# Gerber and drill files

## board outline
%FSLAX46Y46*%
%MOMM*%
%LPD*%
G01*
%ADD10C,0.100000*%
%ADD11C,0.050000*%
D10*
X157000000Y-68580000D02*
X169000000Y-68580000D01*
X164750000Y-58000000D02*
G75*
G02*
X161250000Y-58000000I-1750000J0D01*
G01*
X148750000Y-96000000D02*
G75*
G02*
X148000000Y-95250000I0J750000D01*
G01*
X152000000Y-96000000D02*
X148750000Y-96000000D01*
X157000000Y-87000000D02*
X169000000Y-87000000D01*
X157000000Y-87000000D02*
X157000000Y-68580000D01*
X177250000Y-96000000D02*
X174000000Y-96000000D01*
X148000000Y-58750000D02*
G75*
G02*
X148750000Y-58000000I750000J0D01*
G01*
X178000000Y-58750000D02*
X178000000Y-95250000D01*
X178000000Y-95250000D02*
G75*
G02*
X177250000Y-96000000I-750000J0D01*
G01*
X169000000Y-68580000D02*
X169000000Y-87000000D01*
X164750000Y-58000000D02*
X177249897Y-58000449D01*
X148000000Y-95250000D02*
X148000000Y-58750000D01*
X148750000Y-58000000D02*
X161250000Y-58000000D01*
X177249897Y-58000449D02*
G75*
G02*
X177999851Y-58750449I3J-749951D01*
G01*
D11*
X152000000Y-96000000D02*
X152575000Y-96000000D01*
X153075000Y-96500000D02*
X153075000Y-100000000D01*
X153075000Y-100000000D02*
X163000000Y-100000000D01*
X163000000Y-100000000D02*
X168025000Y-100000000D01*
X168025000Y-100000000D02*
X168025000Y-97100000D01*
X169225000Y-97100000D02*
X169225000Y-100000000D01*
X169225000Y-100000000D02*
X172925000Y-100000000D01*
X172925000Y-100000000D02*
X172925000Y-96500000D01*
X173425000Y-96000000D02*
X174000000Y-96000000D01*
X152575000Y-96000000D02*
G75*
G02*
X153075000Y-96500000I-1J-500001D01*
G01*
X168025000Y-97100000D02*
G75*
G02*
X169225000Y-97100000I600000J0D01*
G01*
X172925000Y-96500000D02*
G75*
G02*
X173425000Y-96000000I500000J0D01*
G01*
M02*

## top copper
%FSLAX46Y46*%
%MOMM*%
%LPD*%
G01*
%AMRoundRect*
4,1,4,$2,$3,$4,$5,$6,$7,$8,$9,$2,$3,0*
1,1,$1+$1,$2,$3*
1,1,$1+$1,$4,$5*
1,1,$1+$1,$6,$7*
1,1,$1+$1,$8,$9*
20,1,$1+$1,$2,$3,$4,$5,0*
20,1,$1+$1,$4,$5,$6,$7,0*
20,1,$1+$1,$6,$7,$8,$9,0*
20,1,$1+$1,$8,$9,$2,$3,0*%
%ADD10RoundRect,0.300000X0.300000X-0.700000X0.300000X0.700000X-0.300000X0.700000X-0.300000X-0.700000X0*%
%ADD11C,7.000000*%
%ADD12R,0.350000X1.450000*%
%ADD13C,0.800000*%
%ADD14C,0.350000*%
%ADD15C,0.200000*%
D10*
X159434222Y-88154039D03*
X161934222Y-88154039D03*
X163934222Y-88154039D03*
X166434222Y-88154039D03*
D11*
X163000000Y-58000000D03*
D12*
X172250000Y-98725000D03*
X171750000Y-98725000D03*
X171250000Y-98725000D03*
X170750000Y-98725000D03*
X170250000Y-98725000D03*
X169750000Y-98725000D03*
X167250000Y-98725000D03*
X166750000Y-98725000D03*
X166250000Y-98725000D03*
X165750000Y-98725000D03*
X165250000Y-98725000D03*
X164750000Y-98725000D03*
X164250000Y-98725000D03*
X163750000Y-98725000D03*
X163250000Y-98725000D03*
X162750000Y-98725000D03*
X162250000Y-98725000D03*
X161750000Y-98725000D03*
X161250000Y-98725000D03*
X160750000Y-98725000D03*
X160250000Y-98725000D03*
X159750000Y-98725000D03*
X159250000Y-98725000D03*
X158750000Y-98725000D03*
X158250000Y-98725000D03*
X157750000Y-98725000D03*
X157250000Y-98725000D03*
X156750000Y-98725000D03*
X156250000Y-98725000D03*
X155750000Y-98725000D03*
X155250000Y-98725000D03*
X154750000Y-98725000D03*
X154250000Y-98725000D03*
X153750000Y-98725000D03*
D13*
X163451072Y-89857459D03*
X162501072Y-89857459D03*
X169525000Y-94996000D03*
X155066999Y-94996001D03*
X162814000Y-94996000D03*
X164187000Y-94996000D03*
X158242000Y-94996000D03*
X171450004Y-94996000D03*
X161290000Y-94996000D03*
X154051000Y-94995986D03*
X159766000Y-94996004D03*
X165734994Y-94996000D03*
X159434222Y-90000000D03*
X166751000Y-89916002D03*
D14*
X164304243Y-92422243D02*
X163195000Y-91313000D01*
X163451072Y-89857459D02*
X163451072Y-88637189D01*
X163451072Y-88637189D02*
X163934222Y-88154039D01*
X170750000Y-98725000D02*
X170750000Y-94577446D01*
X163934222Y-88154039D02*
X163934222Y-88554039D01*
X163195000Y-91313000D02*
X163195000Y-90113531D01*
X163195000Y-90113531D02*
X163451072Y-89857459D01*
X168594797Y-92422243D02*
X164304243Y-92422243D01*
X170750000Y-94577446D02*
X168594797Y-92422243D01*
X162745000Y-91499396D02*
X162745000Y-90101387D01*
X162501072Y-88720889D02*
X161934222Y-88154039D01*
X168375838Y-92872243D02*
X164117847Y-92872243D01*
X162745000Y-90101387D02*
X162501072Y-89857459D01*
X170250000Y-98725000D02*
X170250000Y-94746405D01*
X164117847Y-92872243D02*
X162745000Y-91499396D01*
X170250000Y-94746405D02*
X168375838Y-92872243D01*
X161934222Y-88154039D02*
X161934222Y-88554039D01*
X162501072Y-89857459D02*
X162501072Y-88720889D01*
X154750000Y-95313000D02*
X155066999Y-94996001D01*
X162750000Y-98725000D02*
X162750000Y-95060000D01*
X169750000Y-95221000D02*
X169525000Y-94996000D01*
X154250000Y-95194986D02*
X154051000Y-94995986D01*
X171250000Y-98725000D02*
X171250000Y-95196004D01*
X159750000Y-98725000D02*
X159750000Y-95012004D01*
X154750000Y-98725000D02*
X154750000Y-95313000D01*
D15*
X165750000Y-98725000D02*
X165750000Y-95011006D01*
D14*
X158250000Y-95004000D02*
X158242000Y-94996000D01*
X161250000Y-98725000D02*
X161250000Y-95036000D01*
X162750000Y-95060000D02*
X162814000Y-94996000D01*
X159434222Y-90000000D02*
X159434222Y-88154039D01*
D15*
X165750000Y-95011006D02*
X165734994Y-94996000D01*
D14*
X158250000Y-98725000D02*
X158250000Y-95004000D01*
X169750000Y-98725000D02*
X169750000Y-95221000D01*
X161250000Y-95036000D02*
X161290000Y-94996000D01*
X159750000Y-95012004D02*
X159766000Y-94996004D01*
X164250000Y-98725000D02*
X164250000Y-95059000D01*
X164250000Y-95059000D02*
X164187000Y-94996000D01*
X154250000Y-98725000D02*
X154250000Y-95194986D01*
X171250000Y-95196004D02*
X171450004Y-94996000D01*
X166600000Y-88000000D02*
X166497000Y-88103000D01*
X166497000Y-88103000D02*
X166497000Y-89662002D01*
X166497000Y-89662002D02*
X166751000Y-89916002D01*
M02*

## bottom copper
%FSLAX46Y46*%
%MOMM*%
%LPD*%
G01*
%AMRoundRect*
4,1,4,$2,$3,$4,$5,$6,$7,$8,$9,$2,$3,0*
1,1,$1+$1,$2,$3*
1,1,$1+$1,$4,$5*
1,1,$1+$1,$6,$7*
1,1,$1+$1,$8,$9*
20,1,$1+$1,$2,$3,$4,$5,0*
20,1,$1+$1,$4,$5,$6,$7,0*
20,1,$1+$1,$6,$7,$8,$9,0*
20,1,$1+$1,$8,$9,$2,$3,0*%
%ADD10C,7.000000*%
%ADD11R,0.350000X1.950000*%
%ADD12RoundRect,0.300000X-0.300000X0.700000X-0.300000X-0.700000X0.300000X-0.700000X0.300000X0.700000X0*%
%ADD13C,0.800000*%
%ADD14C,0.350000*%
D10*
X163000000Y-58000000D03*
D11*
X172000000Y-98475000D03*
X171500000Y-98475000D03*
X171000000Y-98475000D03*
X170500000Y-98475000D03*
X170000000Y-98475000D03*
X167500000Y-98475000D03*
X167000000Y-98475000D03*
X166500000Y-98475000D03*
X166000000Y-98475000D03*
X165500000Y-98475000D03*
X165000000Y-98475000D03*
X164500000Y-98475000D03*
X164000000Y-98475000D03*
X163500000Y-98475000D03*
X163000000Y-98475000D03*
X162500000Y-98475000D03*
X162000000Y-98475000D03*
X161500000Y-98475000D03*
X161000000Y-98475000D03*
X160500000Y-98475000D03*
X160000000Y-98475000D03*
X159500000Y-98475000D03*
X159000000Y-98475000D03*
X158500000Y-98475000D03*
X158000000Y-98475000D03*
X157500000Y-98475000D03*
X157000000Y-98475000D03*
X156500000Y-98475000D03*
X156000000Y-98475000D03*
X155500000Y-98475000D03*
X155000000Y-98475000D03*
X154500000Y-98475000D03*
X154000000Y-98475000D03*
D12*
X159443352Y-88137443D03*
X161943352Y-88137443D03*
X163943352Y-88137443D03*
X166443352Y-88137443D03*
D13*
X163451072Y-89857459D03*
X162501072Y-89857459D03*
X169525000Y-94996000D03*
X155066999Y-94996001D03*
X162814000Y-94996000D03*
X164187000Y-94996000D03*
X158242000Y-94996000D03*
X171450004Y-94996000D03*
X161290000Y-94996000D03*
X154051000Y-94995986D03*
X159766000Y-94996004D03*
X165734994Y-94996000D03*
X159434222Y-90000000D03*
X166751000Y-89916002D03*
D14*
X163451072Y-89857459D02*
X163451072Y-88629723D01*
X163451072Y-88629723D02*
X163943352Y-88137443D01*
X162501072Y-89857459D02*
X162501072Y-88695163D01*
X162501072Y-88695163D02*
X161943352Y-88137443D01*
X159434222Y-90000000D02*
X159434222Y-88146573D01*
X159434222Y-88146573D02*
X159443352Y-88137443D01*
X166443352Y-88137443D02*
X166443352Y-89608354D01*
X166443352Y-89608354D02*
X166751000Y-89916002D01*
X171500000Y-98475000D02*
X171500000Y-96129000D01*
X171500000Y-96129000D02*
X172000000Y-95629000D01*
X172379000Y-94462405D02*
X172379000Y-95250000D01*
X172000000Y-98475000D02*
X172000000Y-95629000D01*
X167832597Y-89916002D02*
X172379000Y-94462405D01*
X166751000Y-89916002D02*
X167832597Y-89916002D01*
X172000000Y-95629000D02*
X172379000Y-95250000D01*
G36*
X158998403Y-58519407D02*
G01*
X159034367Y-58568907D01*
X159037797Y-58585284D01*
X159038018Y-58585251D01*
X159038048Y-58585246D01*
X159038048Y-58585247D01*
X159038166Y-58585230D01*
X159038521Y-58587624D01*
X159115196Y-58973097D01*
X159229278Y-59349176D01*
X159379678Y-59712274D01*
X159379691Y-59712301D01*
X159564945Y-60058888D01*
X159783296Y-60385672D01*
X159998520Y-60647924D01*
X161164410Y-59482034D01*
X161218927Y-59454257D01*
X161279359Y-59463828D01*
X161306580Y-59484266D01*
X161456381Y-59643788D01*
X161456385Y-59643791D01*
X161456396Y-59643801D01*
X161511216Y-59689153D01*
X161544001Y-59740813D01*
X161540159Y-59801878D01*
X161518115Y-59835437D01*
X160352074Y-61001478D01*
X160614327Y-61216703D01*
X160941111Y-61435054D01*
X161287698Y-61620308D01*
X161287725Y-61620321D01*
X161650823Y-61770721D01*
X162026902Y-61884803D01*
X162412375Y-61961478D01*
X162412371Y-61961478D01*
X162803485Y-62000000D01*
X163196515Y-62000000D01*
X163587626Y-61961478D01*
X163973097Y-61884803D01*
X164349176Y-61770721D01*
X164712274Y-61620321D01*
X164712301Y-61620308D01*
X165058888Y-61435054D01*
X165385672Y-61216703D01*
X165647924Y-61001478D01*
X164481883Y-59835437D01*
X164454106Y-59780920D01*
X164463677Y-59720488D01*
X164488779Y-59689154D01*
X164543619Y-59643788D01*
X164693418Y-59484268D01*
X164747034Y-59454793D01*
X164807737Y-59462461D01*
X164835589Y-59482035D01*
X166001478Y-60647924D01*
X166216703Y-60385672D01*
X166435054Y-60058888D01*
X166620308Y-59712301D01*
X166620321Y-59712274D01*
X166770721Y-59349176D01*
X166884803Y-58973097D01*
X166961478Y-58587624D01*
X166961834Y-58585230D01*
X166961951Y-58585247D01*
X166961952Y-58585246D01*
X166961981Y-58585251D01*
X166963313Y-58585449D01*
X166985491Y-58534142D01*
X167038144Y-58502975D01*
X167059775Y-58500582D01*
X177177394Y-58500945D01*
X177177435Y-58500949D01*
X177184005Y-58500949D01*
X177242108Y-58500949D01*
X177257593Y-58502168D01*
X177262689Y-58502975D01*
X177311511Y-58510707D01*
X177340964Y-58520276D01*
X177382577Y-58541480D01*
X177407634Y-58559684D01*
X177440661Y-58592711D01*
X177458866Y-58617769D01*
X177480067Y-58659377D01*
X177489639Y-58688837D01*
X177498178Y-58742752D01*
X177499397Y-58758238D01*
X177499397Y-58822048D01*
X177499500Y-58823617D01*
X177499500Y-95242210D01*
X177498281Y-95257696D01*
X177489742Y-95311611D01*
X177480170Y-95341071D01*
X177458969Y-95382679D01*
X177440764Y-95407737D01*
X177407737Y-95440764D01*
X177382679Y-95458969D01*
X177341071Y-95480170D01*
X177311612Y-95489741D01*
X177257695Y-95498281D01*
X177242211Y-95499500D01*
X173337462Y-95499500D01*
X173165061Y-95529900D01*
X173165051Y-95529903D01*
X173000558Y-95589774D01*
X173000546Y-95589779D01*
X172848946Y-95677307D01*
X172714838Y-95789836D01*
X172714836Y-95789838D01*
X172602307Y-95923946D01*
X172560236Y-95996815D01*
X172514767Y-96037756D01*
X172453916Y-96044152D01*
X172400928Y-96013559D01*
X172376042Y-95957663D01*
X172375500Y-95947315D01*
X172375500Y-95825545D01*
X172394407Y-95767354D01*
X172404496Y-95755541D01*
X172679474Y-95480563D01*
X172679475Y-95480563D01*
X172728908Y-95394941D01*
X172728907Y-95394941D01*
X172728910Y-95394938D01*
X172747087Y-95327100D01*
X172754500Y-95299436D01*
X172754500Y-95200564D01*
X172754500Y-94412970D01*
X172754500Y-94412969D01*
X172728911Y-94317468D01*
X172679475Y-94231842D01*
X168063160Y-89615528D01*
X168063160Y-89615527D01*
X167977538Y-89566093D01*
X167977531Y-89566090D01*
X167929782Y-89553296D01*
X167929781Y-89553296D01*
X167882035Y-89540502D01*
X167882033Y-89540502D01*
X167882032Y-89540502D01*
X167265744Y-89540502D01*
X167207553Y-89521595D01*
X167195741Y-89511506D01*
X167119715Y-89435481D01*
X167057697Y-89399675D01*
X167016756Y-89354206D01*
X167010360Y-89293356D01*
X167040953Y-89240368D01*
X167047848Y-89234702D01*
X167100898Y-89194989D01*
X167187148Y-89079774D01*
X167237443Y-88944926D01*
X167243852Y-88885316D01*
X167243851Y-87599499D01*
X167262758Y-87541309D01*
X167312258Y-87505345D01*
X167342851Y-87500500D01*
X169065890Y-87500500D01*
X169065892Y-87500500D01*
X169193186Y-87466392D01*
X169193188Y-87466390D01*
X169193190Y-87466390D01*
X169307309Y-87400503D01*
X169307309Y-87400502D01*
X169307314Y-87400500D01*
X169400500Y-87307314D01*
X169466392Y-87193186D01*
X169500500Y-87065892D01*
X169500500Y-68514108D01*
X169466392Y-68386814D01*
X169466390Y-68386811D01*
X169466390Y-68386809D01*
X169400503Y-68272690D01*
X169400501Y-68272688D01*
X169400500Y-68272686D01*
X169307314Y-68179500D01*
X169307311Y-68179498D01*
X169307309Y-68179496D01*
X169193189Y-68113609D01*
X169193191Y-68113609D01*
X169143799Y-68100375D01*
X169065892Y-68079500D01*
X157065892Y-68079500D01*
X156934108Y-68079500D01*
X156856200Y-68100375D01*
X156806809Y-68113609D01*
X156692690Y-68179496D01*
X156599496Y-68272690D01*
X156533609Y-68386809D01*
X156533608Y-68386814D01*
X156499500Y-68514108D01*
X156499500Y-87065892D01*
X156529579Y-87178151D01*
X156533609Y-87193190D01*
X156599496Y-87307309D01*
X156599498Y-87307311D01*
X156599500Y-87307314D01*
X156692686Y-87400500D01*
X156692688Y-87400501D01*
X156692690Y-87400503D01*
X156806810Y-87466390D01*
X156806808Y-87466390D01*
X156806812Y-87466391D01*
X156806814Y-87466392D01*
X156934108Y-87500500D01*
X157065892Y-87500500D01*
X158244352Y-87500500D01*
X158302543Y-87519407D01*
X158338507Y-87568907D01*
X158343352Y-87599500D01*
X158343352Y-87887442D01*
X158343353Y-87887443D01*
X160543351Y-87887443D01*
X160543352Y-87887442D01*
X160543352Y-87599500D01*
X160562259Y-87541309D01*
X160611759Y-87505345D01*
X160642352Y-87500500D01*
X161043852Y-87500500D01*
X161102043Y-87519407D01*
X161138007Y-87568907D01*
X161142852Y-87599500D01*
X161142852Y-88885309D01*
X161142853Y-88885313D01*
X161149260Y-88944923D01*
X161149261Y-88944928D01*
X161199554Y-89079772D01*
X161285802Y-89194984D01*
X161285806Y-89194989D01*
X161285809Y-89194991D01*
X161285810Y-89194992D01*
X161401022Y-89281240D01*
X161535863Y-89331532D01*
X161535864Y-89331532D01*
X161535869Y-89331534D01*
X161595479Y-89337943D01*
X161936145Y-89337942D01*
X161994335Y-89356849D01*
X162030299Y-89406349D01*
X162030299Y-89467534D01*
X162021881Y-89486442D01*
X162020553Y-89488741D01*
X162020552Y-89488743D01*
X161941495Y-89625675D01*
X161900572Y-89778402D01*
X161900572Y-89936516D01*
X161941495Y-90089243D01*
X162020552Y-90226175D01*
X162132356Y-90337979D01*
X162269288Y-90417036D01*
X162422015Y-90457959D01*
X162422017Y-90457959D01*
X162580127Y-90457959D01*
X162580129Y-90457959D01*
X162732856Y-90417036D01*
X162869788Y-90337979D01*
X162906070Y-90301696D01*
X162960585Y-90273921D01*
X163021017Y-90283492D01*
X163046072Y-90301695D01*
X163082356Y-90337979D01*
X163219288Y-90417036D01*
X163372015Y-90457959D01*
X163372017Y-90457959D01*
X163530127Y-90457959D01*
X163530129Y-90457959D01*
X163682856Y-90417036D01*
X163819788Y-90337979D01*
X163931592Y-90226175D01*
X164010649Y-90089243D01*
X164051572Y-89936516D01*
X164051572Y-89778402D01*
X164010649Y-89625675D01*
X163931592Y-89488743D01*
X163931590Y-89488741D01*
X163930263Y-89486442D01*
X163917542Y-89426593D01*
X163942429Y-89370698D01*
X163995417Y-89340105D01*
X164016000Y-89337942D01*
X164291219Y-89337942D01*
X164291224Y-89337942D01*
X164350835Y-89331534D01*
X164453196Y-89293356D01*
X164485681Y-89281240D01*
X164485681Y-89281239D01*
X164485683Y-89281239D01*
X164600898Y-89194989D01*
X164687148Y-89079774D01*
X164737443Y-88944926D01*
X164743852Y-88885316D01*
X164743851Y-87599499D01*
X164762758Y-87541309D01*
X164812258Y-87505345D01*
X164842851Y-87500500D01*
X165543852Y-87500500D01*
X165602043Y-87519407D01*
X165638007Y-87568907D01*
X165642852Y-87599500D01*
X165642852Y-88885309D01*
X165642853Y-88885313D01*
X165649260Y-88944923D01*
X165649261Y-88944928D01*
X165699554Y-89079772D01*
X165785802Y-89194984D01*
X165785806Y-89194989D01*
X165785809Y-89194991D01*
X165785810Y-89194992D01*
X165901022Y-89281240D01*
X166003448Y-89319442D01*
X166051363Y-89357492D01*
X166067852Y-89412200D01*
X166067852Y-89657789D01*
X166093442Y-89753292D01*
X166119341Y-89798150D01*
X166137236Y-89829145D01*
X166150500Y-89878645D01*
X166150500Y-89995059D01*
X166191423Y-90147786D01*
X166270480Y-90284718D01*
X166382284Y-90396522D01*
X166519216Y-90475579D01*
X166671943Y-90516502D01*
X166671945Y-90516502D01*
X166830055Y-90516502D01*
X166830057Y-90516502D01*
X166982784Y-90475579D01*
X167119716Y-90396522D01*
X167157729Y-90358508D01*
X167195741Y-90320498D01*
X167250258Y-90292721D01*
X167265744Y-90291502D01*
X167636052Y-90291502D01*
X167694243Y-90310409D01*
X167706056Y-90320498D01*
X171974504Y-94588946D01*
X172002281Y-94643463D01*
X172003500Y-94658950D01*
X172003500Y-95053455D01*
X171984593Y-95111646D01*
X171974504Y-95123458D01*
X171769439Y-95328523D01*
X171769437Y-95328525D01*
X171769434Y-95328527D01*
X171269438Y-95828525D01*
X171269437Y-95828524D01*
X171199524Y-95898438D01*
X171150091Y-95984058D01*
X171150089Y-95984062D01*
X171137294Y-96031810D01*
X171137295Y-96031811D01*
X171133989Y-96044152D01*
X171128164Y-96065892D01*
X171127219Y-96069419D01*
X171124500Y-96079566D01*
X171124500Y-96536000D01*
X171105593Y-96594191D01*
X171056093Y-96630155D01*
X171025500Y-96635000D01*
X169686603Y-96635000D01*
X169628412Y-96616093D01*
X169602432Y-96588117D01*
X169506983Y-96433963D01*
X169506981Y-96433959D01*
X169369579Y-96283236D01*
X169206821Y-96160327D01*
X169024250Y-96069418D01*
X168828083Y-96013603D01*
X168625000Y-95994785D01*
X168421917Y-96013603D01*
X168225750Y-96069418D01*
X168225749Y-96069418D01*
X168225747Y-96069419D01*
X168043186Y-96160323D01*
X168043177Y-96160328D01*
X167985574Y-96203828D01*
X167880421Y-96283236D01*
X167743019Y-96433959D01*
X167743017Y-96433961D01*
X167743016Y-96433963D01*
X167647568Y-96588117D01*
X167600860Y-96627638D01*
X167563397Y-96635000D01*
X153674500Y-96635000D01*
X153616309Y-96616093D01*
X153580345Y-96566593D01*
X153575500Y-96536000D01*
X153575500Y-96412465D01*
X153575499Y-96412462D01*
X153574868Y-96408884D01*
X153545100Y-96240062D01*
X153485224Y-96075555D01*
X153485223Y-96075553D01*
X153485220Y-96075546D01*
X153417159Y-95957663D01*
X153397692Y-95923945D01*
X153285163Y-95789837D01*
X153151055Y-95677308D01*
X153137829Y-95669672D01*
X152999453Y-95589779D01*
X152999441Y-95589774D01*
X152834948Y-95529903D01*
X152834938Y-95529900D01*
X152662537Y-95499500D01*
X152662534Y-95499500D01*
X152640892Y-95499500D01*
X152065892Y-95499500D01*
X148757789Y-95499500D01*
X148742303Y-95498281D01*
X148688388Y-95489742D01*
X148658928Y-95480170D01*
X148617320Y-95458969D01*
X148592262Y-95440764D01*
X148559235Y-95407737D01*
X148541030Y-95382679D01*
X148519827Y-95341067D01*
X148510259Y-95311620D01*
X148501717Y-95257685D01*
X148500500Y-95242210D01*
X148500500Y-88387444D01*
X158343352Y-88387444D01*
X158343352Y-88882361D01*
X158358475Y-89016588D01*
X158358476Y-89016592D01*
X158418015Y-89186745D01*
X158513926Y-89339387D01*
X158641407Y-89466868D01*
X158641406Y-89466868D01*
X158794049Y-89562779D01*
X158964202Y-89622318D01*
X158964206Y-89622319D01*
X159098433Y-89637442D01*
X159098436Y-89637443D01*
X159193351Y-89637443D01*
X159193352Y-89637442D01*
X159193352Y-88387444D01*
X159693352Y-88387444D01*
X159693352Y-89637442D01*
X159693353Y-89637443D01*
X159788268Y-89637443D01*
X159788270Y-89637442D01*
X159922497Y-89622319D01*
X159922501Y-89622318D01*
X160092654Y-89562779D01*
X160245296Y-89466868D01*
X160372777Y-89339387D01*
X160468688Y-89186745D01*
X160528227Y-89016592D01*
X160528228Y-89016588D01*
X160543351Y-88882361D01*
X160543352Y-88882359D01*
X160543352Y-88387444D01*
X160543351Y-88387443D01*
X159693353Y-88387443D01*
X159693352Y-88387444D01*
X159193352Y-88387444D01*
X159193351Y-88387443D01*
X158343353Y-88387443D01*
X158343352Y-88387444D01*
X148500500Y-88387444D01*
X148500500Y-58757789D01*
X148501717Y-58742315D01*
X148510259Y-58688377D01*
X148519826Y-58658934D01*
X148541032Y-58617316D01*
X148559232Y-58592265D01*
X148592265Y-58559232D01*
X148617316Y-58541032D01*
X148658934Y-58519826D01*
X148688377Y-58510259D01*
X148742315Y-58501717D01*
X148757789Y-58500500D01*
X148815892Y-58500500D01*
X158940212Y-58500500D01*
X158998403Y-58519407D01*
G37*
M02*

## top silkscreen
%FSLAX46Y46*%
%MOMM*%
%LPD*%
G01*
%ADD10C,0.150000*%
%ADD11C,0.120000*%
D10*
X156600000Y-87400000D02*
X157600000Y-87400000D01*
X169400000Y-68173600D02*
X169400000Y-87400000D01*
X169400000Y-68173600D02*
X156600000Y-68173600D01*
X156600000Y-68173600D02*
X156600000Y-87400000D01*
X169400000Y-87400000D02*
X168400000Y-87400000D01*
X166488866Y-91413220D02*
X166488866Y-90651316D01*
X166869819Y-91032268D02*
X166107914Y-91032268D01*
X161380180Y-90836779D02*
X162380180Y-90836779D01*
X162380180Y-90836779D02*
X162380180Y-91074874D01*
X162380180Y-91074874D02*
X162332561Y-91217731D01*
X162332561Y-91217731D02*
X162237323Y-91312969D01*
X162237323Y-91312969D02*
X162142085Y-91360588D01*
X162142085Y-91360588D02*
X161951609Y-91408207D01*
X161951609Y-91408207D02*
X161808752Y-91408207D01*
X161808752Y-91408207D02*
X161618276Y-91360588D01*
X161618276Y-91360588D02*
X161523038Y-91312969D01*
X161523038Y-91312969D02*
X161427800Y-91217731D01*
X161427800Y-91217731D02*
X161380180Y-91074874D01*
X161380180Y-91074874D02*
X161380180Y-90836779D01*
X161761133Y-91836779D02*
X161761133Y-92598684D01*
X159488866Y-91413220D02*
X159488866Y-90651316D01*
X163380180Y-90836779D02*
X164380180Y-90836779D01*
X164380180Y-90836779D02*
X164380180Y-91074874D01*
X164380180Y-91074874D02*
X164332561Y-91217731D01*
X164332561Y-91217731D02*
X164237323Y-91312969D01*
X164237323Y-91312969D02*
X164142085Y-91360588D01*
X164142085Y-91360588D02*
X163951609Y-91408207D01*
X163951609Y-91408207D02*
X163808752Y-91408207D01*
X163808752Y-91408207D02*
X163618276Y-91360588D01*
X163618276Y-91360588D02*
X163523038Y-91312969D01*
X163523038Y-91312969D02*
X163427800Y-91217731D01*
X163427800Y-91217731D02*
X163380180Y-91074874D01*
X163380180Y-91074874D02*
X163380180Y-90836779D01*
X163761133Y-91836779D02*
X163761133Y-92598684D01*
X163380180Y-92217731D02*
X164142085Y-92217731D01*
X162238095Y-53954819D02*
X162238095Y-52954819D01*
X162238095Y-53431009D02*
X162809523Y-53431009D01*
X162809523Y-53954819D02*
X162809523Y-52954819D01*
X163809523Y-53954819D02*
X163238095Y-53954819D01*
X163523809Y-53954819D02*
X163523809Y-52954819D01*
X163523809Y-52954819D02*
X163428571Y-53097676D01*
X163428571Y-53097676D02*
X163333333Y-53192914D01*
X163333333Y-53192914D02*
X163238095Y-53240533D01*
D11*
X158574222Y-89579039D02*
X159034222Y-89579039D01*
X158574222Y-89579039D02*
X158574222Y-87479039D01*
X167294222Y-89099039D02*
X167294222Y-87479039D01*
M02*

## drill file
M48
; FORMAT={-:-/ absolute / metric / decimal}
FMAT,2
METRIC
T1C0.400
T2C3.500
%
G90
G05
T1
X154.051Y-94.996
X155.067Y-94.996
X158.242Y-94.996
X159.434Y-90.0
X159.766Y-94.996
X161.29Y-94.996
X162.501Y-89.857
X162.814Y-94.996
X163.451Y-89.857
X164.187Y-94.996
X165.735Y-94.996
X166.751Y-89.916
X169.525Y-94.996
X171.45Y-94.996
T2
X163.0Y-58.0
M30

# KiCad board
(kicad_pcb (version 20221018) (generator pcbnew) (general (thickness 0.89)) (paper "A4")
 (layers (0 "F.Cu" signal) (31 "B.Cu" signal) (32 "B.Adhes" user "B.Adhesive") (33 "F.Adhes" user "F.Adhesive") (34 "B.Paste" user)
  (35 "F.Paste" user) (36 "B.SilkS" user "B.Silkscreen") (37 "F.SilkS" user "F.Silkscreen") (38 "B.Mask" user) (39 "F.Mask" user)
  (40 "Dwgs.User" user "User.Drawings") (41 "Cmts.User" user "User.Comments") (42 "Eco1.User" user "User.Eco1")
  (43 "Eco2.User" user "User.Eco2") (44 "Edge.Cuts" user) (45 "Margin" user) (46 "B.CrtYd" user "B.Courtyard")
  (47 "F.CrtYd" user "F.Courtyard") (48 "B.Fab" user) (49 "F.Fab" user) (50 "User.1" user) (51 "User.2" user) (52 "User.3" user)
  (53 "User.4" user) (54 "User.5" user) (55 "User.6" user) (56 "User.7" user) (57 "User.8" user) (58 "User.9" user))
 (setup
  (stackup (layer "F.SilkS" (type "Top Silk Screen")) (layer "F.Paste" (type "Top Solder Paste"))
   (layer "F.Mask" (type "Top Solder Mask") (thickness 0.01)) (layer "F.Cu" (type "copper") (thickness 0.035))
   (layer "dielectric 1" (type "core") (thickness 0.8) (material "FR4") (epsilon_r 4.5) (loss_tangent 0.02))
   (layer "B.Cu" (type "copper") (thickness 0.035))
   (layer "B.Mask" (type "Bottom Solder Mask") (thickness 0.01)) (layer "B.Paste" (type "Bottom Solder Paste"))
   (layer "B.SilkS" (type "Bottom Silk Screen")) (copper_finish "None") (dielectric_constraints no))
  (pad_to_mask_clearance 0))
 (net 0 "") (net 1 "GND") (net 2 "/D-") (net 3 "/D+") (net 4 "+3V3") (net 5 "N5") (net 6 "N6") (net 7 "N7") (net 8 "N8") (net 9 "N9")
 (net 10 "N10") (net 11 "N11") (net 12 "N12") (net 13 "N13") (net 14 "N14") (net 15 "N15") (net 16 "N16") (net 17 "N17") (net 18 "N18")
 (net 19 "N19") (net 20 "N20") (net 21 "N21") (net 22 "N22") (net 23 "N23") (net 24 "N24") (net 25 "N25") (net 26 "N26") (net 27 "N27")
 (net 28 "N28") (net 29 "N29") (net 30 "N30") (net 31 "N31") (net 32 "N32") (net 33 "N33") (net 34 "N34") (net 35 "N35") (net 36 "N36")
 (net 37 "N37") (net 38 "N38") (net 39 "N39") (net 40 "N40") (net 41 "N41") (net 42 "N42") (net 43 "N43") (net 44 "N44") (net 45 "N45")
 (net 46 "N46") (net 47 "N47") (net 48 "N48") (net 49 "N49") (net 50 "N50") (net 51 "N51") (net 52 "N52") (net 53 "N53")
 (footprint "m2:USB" (layer "F.Cu") (at 162.994222 87.979039 90)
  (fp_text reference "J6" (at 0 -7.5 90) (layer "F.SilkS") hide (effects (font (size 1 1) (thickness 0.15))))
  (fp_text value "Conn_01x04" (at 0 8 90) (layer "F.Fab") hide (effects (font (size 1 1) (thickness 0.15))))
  (fp_line (start -1.6 -4.42) (end -1.6 -3.96) (stroke (width 0.12) (type default)) (layer "F.SilkS"))
  (fp_line (start -1.6 -4.42) (end 0.5 -4.42) (stroke (width 0.12) (type default)) (layer "F.SilkS"))
  (fp_line (start -1.12 4.3) (end 0.5 4.3) (stroke (width 0.12) (type default)) (layer "F.SilkS"))
  (pad "1" smd roundrect (at -0.175 -3.56 90) (size 2 1.2) (layers "F.Cu" "F.Paste" "F.Mask") (roundrect_rratio 0.25) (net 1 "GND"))
  (pad "2" smd roundrect (at -0.175 -1.06 90) (size 2 1.2) (layers "F.Cu" "F.Paste" "F.Mask") (roundrect_rratio 0.25) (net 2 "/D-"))
  (pad "3" smd roundrect (at -0.175 0.94 90) (size 2 1.2) (layers "F.Cu" "F.Paste" "F.Mask") (roundrect_rratio 0.25) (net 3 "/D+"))
  (pad "4" smd roundrect (at -0.175 3.44 90) (size 2 1.2) (layers "F.Cu" "F.Paste" "F.Mask") (roundrect_rratio 0.25) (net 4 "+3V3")))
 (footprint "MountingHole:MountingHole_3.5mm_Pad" (layer "F.Cu") (at 163 58)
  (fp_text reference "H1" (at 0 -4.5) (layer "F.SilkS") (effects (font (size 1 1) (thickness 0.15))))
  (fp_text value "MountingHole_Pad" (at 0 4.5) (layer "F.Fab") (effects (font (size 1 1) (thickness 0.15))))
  (pad "1" thru_hole circle (at 0 0) (size 7 7) (drill 3.5) (layers "*.Cu" "*.Mask") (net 1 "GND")))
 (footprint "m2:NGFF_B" (layer "F.Cu") (at 163 100)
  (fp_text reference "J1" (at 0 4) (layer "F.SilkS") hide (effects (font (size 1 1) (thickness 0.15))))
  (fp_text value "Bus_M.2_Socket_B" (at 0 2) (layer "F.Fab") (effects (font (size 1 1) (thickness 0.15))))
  (fp_line (start -11 -4) (end -10.425 -4) (stroke (width 0.05) (type solid)) (layer "Edge.Cuts"))
  (fp_line (start -9.925 -3.5) (end -9.925 0) (stroke (width 0.05) (type solid)) (layer "Edge.Cuts"))
  (fp_line (start -9.925 0) (end 0 0) (stroke (width 0.05) (type solid)) (layer "Edge.Cuts"))
  (fp_line (start 0 0) (end 5.025 0) (stroke (width 0.05) (type solid)) (layer "Edge.Cuts"))
  (fp_line (start 5.025 0) (end 5.025 -2.9) (stroke (width 0.05) (type solid)) (layer "Edge.Cuts"))
  (fp_line (start 6.225 -2.9) (end 6.225 0) (stroke (width 0.05) (type solid)) (layer "Edge.Cuts"))
  (fp_line (start 6.225 0) (end 9.925 0) (stroke (width 0.05) (type solid)) (layer "Edge.Cuts"))
  (fp_line (start 9.925 0) (end 9.925 -3.5) (stroke (width 0.05) (type solid)) (layer "Edge.Cuts"))
  (fp_line (start 10.425 -4) (end 11 -4) (stroke (width 0.05) (type solid)) (layer "Edge.Cuts"))
  (fp_arc (start -10.425 -4) (mid -10.071447 -3.853553) (end -9.925 -3.5) (stroke (width 0.05) (type solid)) (layer "Edge.Cuts"))
  (fp_arc (start 5.025 -2.9) (mid 5.625 -3.5) (end 6.225 -2.9) (stroke (width 0.05) (type solid)) (layer "Edge.Cuts"))
  (fp_arc (start 9.925 -3.5) (mid 10.071447 -3.853553) (end 10.425 -4) (stroke (width 0.05) (type solid)) (layer "Edge.Cuts"))
  (pad "1" smd rect (at 9.25 -1.275) (size 0.35 1.45) (layers "F.Cu") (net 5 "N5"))
  (pad "2" smd rect (at 9 -1.525) (size 0.35 1.95) (layers "B.Cu") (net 4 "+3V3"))
  (pad "3" smd rect (at 8.75 -1.275) (size 0.35 1.45) (layers "F.Cu") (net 1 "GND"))
  (pad "4" smd rect (at 8.5 -1.525) (size 0.35 1.95) (layers "B.Cu") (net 4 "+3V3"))
  (pad "5" smd rect (at 8.25 -1.275) (size 0.35 1.45) (layers "F.Cu") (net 1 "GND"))
  (pad "6" smd rect (at 8 -1.525) (size 0.35 1.95) (layers "B.Cu") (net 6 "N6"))
  (pad "7" smd rect (at 7.75 -1.275) (size 0.35 1.45) (layers "F.Cu") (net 3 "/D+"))
  (pad "8" smd rect (at 7.5 -1.525) (size 0.35 1.95) (layers "B.Cu") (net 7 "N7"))
  (pad "9" smd rect (at 7.25 -1.275) (size 0.35 1.45) (layers "F.Cu") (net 2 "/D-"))
  (pad "10" smd rect (at 7 -1.525) (size 0.35 1.95) (layers "B.Cu") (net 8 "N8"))
  (pad "11" smd rect (at 6.75 -1.275) (size 0.35 1.45) (layers "F.Cu") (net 1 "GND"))
  (pad "20" smd rect (at 4.5 -1.525) (size 0.35 1.95) (layers "B.Cu") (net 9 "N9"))
  (pad "21" smd rect (at 4.25 -1.275) (size 0.35 1.45) (layers "F.Cu") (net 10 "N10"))
  (pad "22" smd rect (at 4 -1.525) (size 0.35 1.95) (layers "B.Cu") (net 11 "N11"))
  (pad "23" smd rect (at 3.75 -1.275) (size 0.35 1.45) (layers "F.Cu") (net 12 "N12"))
  (pad "24" smd rect (at 3.5 -1.525) (size 0.35 1.95) (layers "B.Cu") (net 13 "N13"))
  (pad "25" smd rect (at 3.25 -1.275) (size 0.35 1.45) (layers "F.Cu") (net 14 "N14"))
  (pad "26" smd rect (at 3 -1.525) (size 0.35 1.95) (layers "B.Cu") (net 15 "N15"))
  (pad "27" smd rect (at 2.75 -1.275) (size 0.35 1.45) (layers "F.Cu") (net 1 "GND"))
  (pad "28" smd rect (at 2.5 -1.525) (size 0.35 1.95) (layers "B.Cu") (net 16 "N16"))
  (pad "29" smd rect (at 2.25 -1.275) (size 0.35 1.45) (layers "F.Cu") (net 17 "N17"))
  (pad "30" smd rect (at 2 -1.525) (size 0.35 1.95) (layers "B.Cu") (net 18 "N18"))
  (pad "31" smd rect (at 1.75 -1.275) (size 0.35 1.45) (layers "F.Cu") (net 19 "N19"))
  (pad "32" smd rect (at 1.5 -1.525) (size 0.35 1.95) (layers "B.Cu") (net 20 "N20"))
  (pad "33" smd rect (at 1.25 -1.275) (size 0.35 1.45) (layers "F.Cu") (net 1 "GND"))
  (pad "34" smd rect (at 1 -1.525) (size 0.35 1.95) (layers "B.Cu") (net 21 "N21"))
  (pad "35" smd rect (at 0.75 -1.275) (size 0.35 1.45) (layers "F.Cu") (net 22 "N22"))
  (pad "36" smd rect (at 0.5 -1.525) (size 0.35 1.95) (layers "B.Cu") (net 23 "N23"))
  (pad "37" smd rect (at 0.25 -1.275) (size 0.35 1.45) (layers "F.Cu") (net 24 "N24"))
  (pad "38" smd rect (at 0 -1.525) (size 0.35 1.95) (layers "B.Cu") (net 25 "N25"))
  (pad "39" smd rect (at -0.25 -1.275) (size 0.35 1.45) (layers "F.Cu") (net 1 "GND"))
  (pad "40" smd rect (at -0.5 -1.525) (size 0.35 1.95) (layers "B.Cu") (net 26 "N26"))
  (pad "41" smd rect (at -0.75 -1.275) (size 0.35 1.45) (layers "F.Cu") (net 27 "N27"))
  (pad "42" smd rect (at -1 -1.525) (size 0.35 1.95) (layers "B.Cu") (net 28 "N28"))
  (pad "43" smd rect (at -1.25 -1.275) (size 0.35 1.45) (layers "F.Cu") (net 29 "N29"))
  (pad "44" smd rect (at -1.5 -1.525) (size 0.35 1.95) (layers "B.Cu") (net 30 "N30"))
  (pad "45" smd rect (at -1.75 -1.275) (size 0.35 1.45) (layers "F.Cu") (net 1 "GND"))
  (pad "46" smd rect (at -2 -1.525) (size 0.35 1.95) (layers "B.Cu") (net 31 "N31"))
  (pad "47" smd rect (at -2.25 -1.275) (size 0.35 1.45) (layers "F.Cu") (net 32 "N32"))
  (pad "48" smd rect (at -2.5 -1.525) (size 0.35 1.95) (layers "B.Cu") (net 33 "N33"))
  (pad "49" smd rect (at -2.75 -1.275) (size 0.35 1.45) (layers "F.Cu") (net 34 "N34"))
  (pad "50" smd rect (at -3 -1.525) (size 0.35 1.95) (layers "B.Cu") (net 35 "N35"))
  (pad "51" smd rect (at -3.25 -1.275) (size 0.35 1.45) (layers "F.Cu") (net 1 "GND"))
  (pad "52" smd rect (at -3.5 -1.525) (size 0.35 1.95) (layers "B.Cu") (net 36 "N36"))
  (pad "53" smd rect (at -3.75 -1.275) (size 0.35 1.45) (layers "F.Cu") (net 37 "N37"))
  (pad "54" smd rect (at -4 -1.525) (size 0.35 1.95) (layers "B.Cu") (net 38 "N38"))
  (pad "55" smd rect (at -4.25 -1.275) (size 0.35 1.45) (layers "F.Cu") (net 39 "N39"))
  (pad "56" smd rect (at -4.5 -1.525) (size 0.35 1.95) (layers "B.Cu") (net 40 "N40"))
  (pad "57" smd rect (at -4.75 -1.275) (size 0.35 1.45) (layers "F.Cu") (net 1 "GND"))
  (pad "58" smd rect (at -5 -1.525) (size 0.35 1.95) (layers "B.Cu") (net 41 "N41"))
  (pad "59" smd rect (at -5.25 -1.275) (size 0.35 1.45) (layers "F.Cu") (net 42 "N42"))
  (pad "60" smd rect (at -5.5 -1.525) (size 0.35 1.95) (layers "B.Cu") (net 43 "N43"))
  (pad "61" smd rect (at -5.75 -1.275) (size 0.35 1.45) (layers "F.Cu") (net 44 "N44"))
  (pad "62" smd rect (at -6 -1.525) (size 0.35 1.95) (layers "B.Cu") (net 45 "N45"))
  (pad "63" smd rect (at -6.25 -1.275) (size 0.35 1.45) (layers "F.Cu") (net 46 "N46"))
  (pad "64" smd rect (at -6.5 -1.525) (size 0.35 1.95) (layers "B.Cu") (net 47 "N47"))
  (pad "65" smd rect (at -6.75 -1.275) (size 0.35 1.45) (layers "F.Cu") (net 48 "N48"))
  (pad "66" smd rect (at -7 -1.525) (size 0.35 1.95) (layers "B.Cu") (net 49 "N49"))
  (pad "67" smd rect (at -7.25 -1.275) (size 0.35 1.45) (layers "F.Cu") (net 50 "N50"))
  (pad "68" smd rect (at -7.5 -1.525) (size 0.35 1.95) (layers "B.Cu") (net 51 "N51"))
  (pad "69" smd rect (at -7.75 -1.275) (size 0.35 1.45) (layers "F.Cu") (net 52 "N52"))
  (pad "70" smd rect (at -8 -1.525) (size 0.35 1.95) (layers "B.Cu") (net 4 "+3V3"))
  (pad "71" smd rect (at -8.25 -1.275) (size 0.35 1.45) (layers "F.Cu") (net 1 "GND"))
  (pad "72" smd rect (at -8.5 -1.525) (size 0.35 1.95) (layers "B.Cu") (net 4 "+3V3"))
  (pad "73" smd rect (at -8.75 -1.275) (size 0.35 1.45) (layers "F.Cu") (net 1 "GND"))
  (pad "74" smd rect (at -9 -1.525) (size 0.35 1.95) (layers "B.Cu") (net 4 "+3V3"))
  (pad "75" smd rect (at -9.25 -1.275) (size 0.35 1.45) (layers "F.Cu") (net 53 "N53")))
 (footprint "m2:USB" (layer "B.Cu") (at 163.003352 88.312443 -90)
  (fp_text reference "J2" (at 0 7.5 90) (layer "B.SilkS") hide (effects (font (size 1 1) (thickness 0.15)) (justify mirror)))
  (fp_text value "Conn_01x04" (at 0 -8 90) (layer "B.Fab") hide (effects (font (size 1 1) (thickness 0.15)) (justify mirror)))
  (pad "1" smd roundrect (at -0.175 3.56 270) (size 2 1.2) (layers "B.Cu" "B.Paste" "B.Mask") (roundrect_rratio 0.25) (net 1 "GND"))
  (pad "2" smd roundrect (at -0.175 1.06 270) (size 2 1.2) (layers "B.Cu" "B.Paste" "B.Mask") (roundrect_rratio 0.25) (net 2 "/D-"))
  (pad "3" smd roundrect (at -0.175 -0.94 270) (size 2 1.2) (layers "B.Cu" "B.Paste" "B.Mask") (roundrect_rratio 0.25) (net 3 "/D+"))
  (pad "4" smd roundrect (at -0.175 -3.44 270) (size 2 1.2) (layers "B.Cu" "B.Paste" "B.Mask") (roundrect_rratio 0.25) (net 4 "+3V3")))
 (gr_line (start 156.6 87.4) (end 157.6 87.4) (stroke (width 0.15) (type default)) (layer "F.SilkS"))
 (gr_line (start 169.4 68.1736) (end 169.4 87.4) (stroke (width 0.15) (type default)) (layer "F.SilkS"))
 (gr_line (start 169.4 68.1736) (end 156.6 68.1736) (stroke (width 0.15) (type default)) (layer "F.SilkS"))
 (gr_line (start 156.6 68.1736) (end 156.6 87.4) (stroke (width 0.15) (type default)) (layer "F.SilkS"))
 (gr_line (start 169.4 87.4) (end 168.4 87.4) (stroke (width 0.15) (type default)) (layer "F.SilkS"))
 (gr_line (start 157 68.58) (end 169 68.58) (stroke (width 0.1) (type default)) (layer "Edge.Cuts"))
 (gr_arc (start 164.75 58) (mid 163 59.75) (end 161.25 58) (stroke (width 0.1) (type default)) (layer "Edge.Cuts"))
 (gr_arc (start 148.75 96) (mid 148.21967 95.78033) (end 148 95.25) (stroke (width 0.1) (type default)) (layer "Edge.Cuts"))
 (gr_line (start 152 96) (end 148.75 96) (stroke (width 0.1) (type default)) (layer "Edge.Cuts"))
 (gr_line (start 157 87) (end 169 87) (stroke (width 0.1) (type default)) (layer "Edge.Cuts"))
 (gr_line (start 157 87) (end 157 68.58) (stroke (width 0.1) (type default)) (layer "Edge.Cuts"))
 (gr_line (start 177.25 96) (end 174 96) (stroke (width 0.1) (type default)) (layer "Edge.Cuts"))
 (gr_arc (start 148 58.75) (mid 148.21967 58.21967) (end 148.75 58) (stroke (width 0.1) (type default)) (layer "Edge.Cuts"))
 (gr_line (start 178 58.75) (end 178 95.25) (stroke (width 0.1) (type default)) (layer "Edge.Cuts"))
 (gr_arc (start 178 95.25) (mid 177.78033 95.78033) (end 177.25 96) (stroke (width 0.1) (type default)) (layer "Edge.Cuts"))
 (gr_line (start 169 68.58) (end 169 87) (stroke (width 0.1) (type default)) (layer "Edge.Cuts"))
 (gr_line (start 164.75 58) (end 177.249897 58.000449) (stroke (width 0.1) (type default)) (layer "Edge.Cuts"))
 (gr_line (start 148 95.25) (end 148 58.75) (stroke (width 0.1) (type default)) (layer "Edge.Cuts"))
 (gr_line (start 148.75 58) (end 161.25 58) (stroke (width 0.1) (type default)) (layer "Edge.Cuts"))
 (gr_arc (start 177.249897 58.000449) (mid 177.780227 58.220119) (end 177.999897 58.750449) (stroke (width 0.1) (type default))
  (layer "Edge.Cuts"))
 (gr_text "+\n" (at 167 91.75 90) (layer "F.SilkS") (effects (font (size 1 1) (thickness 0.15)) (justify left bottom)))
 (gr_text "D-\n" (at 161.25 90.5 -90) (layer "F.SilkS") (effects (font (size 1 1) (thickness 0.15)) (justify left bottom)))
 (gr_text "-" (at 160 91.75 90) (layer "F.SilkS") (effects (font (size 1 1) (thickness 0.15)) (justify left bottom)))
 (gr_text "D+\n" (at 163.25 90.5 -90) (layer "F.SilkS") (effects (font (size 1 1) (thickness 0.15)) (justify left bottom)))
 (segment (start 164.304243 92.422243) (end 163.195 91.313) (width 0.35) (layer "F.Cu") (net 3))
 (segment (start 163.451072 89.857459) (end 163.451072 88.637189) (width 0.35) (layer "F.Cu") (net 3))
 (segment (start 163.451072 88.637189) (end 163.934222 88.154039) (width 0.35) (layer "F.Cu") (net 3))
 (segment (start 170.75 98.725) (end 170.75 94.577446) (width 0.35) (layer "F.Cu") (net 3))
 (segment (start 163.934222 88.154039) (end 163.934222 88.554039) (width 0.35) (layer "F.Cu") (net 3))
 (segment (start 163.195 91.313) (end 163.195 90.113531) (width 0.35) (layer "F.Cu") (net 3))
 (segment (start 163.195 90.113531) (end 163.451072 89.857459) (width 0.35) (layer "F.Cu") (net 3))
 (segment (start 168.594797 92.422243) (end 164.304243 92.422243) (width 0.35) (layer "F.Cu") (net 3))
 (segment (start 170.75 94.577446) (end 168.594797 92.422243) (width 0.35) (layer "F.Cu") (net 3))
 (via (at 163.451072 89.857459) (size 0.8) (drill 0.4) (layers "F.Cu" "B.Cu") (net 3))
 (segment (start 163.451072 89.857459) (end 163.451072 88.629723) (width 0.35) (layer "B.Cu") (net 3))
 (segment (start 163.451072 88.629723) (end 163.943352 88.137443) (width 0.35) (layer "B.Cu") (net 3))
 (segment (start 162.745 91.499396) (end 162.745 90.101387) (width 0.35) (layer "F.Cu") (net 2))
 (segment (start 162.501072 88.720889) (end 161.934222 88.154039) (width 0.35) (layer "F.Cu") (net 2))
 (segment (start 168.375838 92.872243) (end 164.117847 92.872243) (width 0.35) (layer "F.Cu") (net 2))
 (segment (start 162.745 90.101387) (end 162.501072 89.857459) (width 0.35) (layer "F.Cu") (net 2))
 (segment (start 170.25 98.725) (end 170.25 94.746405) (width 0.35) (layer "F.Cu") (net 2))
 (segment (start 164.117847 92.872243) (end 162.745 91.499396) (width 0.35) (layer "F.Cu") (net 2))
 (segment (start 170.25 94.746405) (end 168.375838 92.872243) (width 0.35) (layer "F.Cu") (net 2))
 (segment (start 161.934222 88.154039) (end 161.934222 88.554039) (width 0.35) (layer "F.Cu") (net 2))
 (segment (start 162.501072 89.857459) (end 162.501072 88.720889) (width 0.35) (layer "F.Cu") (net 2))
 (via (at 162.501072 89.857459) (size 0.8) (drill 0.4) (layers "F.Cu" "B.Cu") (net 2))
 (segment (start 162.501072 89.857459) (end 162.501072 88.695163) (width 0.35) (layer "B.Cu") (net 2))
 (segment (start 162.501072 88.695163) (end 161.943352 88.137443) (width 0.35) (layer "B.Cu") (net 2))
 (segment (start 154.75 95.313) (end 155.066999 94.996001) (width 0.35) (layer "F.Cu") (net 1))
 (segment (start 162.75 98.725) (end 162.75 95.06) (width 0.35) (layer "F.Cu") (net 1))
 (segment (start 169.75 95.221) (end 169.525 94.996) (width 0.35) (layer "F.Cu") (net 1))
 (segment (start 154.25 95.194986) (end 154.051 94.995986) (width 0.35) (layer "F.Cu") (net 1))
 (segment (start 171.25 98.725) (end 171.25 95.196004) (width 0.35) (layer "F.Cu") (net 1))
 (segment (start 159.75 98.725) (end 159.75 95.012004) (width 0.35) (layer "F.Cu") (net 1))
 (segment (start 154.75 98.725) (end 154.75 95.313) (width 0.35) (layer "F.Cu") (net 1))
 (segment (start 165.75 98.725) (end 165.75 95.011006) (width 0.2) (layer "F.Cu") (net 1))
 (segment (start 158.25 95.004) (end 158.242 94.996) (width 0.35) (layer "F.Cu") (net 1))
 (segment (start 161.25 98.725) (end 161.25 95.036) (width 0.35) (layer "F.Cu") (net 1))
 (segment (start 162.75 95.06) (end 162.814 94.996) (width 0.35) (layer "F.Cu") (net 1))
 (segment (start 159.434222 90) (end 159.434222 88.154039) (width 0.35) (layer "F.Cu") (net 1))
 (segment (start 165.75 95.011006) (end 165.734994 94.996) (width 0.2) (layer "F.Cu") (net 1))
 (segment (start 158.25 98.725) (end 158.25 95.004) (width 0.35) (layer "F.Cu") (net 1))
 (segment (start 169.75 98.725) (end 169.75 95.221) (width 0.35) (layer "F.Cu") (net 1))
 (segment (start 161.25 95.036) (end 161.29 94.996) (width 0.35) (layer "F.Cu") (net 1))
 (segment (start 159.75 95.012004) (end 159.766 94.996004) (width 0.35) (layer "F.Cu") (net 1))
 (segment (start 164.25 98.725) (end 164.25 95.059) (width 0.35) (layer "F.Cu") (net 1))
 (segment (start 164.25 95.059) (end 164.187 94.996) (width 0.35) (layer "F.Cu") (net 1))
 (segment (start 154.25 98.725) (end 154.25 95.194986) (width 0.35) (layer "F.Cu") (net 1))
 (segment (start 171.25 95.196004) (end 171.450004 94.996) (width 0.35) (layer "F.Cu") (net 1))
 (via (at 169.525 94.996) (size 0.8) (drill 0.4) (layers "F.Cu" "B.Cu") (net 1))
 (via (at 155.066999 94.996001) (size 0.8) (drill 0.4) (layers "F.Cu" "B.Cu") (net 1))
 (via (at 162.814 94.996) (size 0.8) (drill 0.4) (layers "F.Cu" "B.Cu") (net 1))
 (via (at 164.187 94.996) (size 0.8) (drill 0.4) (layers "F.Cu" "B.Cu") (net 1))
 (via (at 158.242 94.996) (size 0.8) (drill 0.4) (layers "F.Cu" "B.Cu") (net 1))
 (via (at 171.450004 94.996) (size 0.8) (drill 0.4) (layers "F.Cu" "B.Cu") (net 1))
 (via (at 161.29 94.996) (size 0.8) (drill 0.4) (layers "F.Cu" "B.Cu") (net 1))
 (via (at 154.051 94.995986) (size 0.8) (drill 0.4) (layers "F.Cu" "B.Cu") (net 1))
 (via (at 159.766 94.996004) (size 0.8) (drill 0.4) (layers "F.Cu" "B.Cu") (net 1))
 (via (at 165.734994 94.996) (size 0.8) (drill 0.4) (layers "F.Cu" "B.Cu") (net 1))
 (via (at 159.434222 90) (size 0.8) (drill 0.4) (layers "F.Cu" "B.Cu") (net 1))
 (segment (start 159.434222 90) (end 159.434222 88.146573) (width 0.35) (layer "B.Cu") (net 1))
 (segment (start 159.434222 88.146573) (end 159.443352 88.137443) (width 0.35) (layer "B.Cu") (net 1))
 (segment (start 166.6 88) (end 166.497 88.103) (width 0.35) (layer "F.Cu") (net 4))
 (segment (start 166.497 88.103) (end 166.497 89.662002) (width 0.35) (layer "F.Cu") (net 4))
 (segment (start 166.497 89.662002) (end 166.751 89.916002) (width 0.35) (layer "F.Cu") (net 4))
 (via (at 166.751 89.916002) (size 0.8) (drill 0.4) (layers "F.Cu" "B.Cu") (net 4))
 (segment (start 166.443352 88.137443) (end 166.443352 89.608354) (width 0.35) (layer "B.Cu") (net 4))
 (segment (start 166.443352 89.608354) (end 166.751 89.916002) (width 0.35) (layer "B.Cu") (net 4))
 (segment (start 171.5 98.475) (end 171.5 96.129) (width 0.35) (layer "B.Cu") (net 4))
 (segment (start 171.5 96.129) (end 172 95.629) (width 0.35) (layer "B.Cu") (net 4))
 (segment (start 172.379 94.462405) (end 172.379 95.25) (width 0.35) (layer "B.Cu") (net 4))
 (segment (start 172 98.475) (end 172 95.629) (width 0.35) (layer "B.Cu") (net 4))
 (segment (start 167.832597 89.916002) (end 172.379 94.462405) (width 0.35) (layer "B.Cu") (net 4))
 (segment (start 166.751 89.916002) (end 167.832597 89.916002) (width 0.35) (layer "B.Cu") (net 4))
 (segment (start 172 95.629) (end 172.379 95.25) (width 0.35) (layer "B.Cu") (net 4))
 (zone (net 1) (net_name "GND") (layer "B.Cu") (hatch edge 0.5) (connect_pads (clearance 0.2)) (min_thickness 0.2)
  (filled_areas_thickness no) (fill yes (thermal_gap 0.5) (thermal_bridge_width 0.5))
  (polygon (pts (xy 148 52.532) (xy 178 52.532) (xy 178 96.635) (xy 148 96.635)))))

